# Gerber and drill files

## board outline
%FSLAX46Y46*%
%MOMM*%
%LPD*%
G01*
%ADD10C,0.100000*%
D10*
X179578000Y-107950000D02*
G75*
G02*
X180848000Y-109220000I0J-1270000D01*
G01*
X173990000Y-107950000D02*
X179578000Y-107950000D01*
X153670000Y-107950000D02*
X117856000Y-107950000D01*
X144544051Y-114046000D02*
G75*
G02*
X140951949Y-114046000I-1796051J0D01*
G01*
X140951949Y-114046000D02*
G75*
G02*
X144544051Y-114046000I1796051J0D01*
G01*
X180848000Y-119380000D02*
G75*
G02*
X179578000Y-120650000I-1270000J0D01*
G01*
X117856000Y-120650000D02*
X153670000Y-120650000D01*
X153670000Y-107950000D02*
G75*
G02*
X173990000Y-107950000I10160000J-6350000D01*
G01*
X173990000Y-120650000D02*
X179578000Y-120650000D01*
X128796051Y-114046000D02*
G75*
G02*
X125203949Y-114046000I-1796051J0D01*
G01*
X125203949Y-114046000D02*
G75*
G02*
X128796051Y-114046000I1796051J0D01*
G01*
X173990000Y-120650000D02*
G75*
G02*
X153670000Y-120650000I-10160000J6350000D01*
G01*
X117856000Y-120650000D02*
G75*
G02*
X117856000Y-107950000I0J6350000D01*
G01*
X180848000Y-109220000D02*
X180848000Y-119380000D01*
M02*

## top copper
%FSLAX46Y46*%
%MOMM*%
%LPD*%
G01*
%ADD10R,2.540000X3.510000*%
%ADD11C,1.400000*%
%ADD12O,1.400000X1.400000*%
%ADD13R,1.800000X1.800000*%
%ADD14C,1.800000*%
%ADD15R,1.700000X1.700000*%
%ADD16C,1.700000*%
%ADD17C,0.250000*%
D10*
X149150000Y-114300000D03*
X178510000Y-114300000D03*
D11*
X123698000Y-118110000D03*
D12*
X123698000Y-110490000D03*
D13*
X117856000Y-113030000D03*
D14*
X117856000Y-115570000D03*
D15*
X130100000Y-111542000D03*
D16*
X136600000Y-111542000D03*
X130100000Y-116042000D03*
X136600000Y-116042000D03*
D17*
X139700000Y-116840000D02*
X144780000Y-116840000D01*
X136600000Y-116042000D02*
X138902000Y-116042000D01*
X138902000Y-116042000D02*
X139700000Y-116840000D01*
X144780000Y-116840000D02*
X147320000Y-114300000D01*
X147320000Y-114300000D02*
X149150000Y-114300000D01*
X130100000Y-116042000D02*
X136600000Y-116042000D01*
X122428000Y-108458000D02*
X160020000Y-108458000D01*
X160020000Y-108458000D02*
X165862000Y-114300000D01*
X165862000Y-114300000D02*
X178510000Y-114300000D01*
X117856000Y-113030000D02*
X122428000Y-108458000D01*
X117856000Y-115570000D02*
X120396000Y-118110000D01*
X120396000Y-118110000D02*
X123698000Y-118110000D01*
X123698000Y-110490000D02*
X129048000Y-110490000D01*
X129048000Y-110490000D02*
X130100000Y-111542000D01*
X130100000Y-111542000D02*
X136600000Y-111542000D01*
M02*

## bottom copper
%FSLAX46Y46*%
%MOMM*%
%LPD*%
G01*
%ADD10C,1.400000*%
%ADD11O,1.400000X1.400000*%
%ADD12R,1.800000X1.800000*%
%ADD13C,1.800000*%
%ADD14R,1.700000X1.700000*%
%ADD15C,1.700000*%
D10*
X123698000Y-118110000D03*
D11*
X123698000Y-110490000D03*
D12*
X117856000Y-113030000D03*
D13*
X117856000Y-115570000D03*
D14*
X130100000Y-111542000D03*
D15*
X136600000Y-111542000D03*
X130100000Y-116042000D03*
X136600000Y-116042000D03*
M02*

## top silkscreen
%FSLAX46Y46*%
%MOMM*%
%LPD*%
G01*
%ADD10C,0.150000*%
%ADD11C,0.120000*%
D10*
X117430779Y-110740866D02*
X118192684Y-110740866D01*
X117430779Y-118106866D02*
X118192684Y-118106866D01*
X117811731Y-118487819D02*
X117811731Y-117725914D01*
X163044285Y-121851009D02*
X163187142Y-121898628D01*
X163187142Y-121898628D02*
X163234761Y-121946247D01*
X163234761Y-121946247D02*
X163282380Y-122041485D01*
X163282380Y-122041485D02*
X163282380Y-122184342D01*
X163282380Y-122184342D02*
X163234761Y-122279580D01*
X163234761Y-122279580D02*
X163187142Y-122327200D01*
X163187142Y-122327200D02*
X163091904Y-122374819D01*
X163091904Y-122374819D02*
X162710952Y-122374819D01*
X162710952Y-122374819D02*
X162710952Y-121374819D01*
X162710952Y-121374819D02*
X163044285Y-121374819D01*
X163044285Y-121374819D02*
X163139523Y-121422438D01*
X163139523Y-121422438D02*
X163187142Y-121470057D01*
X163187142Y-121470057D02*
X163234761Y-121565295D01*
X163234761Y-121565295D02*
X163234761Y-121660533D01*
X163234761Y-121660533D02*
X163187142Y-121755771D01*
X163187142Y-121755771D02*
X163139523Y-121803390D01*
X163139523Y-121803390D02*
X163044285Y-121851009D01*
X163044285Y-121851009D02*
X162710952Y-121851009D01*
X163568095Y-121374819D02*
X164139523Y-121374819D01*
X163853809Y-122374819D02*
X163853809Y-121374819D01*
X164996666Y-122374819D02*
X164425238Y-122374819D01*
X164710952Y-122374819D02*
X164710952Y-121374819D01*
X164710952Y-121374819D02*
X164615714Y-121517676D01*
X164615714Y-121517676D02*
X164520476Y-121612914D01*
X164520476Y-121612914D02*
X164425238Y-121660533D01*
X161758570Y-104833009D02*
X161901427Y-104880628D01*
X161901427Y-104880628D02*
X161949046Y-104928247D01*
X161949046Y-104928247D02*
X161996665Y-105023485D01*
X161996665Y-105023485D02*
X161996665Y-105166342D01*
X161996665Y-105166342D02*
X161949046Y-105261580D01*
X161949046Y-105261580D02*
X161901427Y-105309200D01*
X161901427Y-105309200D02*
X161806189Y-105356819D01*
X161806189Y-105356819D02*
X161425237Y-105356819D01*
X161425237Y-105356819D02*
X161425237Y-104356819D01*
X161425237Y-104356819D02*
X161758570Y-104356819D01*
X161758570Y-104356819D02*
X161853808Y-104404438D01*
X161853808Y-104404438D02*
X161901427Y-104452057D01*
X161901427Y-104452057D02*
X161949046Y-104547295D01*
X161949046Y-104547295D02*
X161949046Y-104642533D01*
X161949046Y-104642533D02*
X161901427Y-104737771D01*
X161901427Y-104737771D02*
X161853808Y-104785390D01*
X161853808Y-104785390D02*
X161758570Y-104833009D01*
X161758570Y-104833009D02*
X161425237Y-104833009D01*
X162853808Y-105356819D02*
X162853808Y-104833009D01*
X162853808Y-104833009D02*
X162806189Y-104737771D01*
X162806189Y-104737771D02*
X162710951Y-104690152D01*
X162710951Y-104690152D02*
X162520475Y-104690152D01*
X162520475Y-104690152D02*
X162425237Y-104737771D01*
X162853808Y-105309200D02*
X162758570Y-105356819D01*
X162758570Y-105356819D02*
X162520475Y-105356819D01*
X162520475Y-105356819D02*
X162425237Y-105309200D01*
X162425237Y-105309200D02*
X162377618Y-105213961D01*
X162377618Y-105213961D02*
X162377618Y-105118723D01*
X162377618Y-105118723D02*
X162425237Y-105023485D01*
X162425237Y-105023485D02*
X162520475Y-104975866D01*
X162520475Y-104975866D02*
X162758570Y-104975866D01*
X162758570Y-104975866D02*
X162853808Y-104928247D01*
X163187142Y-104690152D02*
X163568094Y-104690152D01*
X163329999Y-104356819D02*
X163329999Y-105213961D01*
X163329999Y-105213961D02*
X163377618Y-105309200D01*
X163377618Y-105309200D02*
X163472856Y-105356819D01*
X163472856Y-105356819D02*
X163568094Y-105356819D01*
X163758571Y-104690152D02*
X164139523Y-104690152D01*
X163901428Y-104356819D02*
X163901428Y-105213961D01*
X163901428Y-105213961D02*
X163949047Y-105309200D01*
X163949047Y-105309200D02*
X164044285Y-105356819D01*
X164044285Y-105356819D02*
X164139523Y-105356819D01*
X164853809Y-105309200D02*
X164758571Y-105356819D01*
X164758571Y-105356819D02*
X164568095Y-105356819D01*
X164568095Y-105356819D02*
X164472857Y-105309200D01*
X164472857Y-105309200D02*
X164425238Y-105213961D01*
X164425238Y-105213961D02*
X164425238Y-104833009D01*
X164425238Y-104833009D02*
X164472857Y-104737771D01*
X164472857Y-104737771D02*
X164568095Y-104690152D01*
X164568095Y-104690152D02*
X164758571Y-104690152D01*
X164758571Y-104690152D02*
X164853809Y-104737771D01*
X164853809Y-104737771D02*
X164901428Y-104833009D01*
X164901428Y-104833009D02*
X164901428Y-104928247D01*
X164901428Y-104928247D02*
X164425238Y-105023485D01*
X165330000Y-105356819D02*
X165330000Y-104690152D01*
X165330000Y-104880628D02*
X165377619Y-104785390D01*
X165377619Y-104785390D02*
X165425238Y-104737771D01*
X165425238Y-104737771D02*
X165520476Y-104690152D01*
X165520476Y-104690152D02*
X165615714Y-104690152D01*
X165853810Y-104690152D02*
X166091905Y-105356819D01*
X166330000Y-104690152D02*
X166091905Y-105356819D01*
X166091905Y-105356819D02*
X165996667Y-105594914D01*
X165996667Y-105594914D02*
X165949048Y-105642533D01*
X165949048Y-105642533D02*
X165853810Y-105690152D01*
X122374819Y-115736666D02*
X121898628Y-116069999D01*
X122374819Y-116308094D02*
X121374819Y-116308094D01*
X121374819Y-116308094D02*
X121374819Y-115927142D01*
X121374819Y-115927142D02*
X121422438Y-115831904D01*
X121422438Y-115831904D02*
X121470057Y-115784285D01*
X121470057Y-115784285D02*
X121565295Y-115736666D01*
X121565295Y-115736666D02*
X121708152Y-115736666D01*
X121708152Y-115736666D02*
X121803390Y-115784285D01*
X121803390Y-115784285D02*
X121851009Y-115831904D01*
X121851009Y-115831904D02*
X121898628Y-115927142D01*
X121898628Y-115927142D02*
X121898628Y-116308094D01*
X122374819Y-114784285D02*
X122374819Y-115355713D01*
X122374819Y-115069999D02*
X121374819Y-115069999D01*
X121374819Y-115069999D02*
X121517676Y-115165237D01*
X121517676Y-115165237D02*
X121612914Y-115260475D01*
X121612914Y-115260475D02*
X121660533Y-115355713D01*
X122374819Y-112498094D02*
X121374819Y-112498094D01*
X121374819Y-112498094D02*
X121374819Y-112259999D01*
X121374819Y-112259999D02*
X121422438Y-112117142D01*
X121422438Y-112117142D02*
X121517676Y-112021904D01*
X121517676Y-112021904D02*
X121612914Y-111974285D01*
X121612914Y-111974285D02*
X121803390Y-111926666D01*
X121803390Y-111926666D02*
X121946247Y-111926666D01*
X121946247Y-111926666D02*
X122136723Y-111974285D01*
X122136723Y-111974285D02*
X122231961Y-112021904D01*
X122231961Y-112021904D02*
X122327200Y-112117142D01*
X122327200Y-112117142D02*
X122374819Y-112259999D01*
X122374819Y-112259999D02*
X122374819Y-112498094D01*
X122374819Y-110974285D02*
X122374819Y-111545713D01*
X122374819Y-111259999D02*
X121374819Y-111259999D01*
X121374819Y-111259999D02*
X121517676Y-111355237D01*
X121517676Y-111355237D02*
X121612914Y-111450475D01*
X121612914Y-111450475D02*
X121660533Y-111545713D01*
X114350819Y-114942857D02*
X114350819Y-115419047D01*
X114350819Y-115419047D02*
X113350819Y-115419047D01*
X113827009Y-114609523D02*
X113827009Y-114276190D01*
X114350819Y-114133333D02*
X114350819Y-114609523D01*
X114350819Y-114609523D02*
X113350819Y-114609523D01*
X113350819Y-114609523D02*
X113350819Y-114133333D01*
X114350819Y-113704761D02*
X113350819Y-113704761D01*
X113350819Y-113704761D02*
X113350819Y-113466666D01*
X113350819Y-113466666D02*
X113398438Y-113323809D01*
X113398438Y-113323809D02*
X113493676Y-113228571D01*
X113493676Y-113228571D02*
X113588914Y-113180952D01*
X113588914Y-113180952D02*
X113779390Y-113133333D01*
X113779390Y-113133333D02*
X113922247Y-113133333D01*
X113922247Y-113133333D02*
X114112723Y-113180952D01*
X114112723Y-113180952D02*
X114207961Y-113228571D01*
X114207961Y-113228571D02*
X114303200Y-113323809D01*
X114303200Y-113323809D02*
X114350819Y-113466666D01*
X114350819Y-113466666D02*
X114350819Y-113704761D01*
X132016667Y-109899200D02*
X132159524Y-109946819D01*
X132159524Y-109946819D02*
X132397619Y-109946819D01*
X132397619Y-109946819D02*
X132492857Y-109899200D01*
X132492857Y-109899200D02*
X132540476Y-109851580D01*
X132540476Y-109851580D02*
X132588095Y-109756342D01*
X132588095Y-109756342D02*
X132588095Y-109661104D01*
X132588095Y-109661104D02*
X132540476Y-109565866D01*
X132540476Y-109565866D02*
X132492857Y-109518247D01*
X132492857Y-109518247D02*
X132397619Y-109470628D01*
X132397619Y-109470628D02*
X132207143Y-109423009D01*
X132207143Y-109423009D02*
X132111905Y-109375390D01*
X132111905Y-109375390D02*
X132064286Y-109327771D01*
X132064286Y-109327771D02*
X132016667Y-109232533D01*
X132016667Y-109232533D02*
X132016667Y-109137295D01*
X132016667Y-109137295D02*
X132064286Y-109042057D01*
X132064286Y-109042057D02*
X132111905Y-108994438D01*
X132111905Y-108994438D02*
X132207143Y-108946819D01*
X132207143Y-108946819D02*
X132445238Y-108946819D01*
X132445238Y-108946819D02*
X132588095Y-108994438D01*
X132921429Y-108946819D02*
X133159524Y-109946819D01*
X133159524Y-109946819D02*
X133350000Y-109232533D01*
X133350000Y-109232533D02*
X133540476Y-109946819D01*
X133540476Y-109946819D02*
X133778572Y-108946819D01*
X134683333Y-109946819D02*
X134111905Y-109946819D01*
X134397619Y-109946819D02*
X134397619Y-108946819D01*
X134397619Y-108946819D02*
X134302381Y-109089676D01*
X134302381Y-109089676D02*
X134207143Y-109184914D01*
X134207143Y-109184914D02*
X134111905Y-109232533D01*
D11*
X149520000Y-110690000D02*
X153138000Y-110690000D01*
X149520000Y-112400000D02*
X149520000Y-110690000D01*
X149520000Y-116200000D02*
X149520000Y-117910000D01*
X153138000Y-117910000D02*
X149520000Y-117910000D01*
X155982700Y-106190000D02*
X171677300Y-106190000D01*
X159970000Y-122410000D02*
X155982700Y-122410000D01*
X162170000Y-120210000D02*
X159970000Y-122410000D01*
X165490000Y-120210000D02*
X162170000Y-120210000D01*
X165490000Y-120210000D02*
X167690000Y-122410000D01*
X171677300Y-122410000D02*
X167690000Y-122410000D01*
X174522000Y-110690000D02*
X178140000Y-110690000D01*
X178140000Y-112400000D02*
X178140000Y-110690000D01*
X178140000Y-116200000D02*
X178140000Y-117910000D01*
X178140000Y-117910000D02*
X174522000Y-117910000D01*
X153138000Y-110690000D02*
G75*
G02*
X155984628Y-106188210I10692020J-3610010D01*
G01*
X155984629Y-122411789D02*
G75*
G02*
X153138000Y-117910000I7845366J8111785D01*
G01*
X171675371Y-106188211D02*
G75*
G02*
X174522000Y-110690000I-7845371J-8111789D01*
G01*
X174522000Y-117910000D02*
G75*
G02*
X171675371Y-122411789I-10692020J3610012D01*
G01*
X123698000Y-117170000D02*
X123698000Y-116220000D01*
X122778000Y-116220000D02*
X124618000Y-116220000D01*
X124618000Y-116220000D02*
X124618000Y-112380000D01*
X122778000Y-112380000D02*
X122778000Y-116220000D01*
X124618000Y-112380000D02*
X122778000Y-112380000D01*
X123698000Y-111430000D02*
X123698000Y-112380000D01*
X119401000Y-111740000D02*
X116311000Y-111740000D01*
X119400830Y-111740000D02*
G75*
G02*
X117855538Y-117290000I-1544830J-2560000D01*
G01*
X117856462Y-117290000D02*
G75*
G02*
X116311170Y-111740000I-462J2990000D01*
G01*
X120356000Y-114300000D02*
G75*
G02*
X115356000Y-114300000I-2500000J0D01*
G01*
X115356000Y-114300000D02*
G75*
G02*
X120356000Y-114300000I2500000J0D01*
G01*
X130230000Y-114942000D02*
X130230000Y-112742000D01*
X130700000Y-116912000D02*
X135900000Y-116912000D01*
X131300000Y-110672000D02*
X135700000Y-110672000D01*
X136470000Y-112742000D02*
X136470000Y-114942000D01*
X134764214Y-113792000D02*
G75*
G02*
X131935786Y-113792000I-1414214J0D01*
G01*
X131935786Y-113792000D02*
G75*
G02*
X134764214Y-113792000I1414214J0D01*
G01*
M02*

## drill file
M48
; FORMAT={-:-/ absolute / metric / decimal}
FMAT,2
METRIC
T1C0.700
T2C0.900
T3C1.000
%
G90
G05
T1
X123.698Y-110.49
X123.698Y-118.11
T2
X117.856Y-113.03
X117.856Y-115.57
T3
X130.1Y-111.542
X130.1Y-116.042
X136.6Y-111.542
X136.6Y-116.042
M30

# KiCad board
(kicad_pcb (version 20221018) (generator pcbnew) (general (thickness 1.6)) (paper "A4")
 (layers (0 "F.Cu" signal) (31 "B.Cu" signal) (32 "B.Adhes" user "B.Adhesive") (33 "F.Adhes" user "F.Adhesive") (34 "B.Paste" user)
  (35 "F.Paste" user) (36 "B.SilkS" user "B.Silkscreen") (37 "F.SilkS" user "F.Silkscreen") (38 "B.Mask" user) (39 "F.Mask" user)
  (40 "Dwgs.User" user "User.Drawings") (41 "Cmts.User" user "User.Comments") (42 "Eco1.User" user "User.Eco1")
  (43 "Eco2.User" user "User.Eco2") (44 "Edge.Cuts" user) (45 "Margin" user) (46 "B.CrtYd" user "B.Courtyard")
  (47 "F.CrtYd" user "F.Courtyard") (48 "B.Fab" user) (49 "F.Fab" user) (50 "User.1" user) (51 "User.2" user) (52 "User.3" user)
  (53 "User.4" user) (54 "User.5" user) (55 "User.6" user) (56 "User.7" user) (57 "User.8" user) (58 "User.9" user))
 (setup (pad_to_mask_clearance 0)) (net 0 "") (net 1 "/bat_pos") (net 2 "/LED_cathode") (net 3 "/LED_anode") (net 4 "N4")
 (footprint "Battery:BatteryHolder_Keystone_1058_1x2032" (layer "F.Cu") (at 163.83 114.3)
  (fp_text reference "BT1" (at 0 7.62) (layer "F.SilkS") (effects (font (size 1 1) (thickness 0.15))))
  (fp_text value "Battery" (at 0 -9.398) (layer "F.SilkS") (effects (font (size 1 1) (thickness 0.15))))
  (fp_line (start -14.31 -3.61) (end -10.692 -3.61) (stroke (width 0.12) (type solid)) (layer "F.SilkS"))
  (fp_line (start -14.31 -1.9) (end -14.31 -3.61) (stroke (width 0.12) (type solid)) (layer "F.SilkS"))
  (fp_line (start -14.31 1.9) (end -14.31 3.61) (stroke (width 0.12) (type solid)) (layer "F.SilkS"))
  (fp_line (start -10.692 3.61) (end -14.31 3.61) (stroke (width 0.12) (type solid)) (layer "F.SilkS"))
  (fp_line (start -7.8473 -8.11) (end 7.8473 -8.11) (stroke (width 0.12) (type solid)) (layer "F.SilkS"))
  (fp_line (start -3.86 8.11) (end -7.8473 8.11) (stroke (width 0.12) (type solid)) (layer "F.SilkS"))
  (fp_line (start -1.66 5.91) (end -3.86 8.11) (stroke (width 0.12) (type solid)) (layer "F.SilkS"))
  (fp_line (start 1.66 5.91) (end -1.66 5.91) (stroke (width 0.12) (type solid)) (layer "F.SilkS"))
  (fp_line (start 1.66 5.91) (end 3.86 8.11) (stroke (width 0.12) (type solid)) (layer "F.SilkS"))
  (fp_line (start 7.8473 8.11) (end 3.86 8.11) (stroke (width 0.12) (type solid)) (layer "F.SilkS"))
  (fp_line (start 10.692 -3.61) (end 14.31 -3.61) (stroke (width 0.12) (type solid)) (layer "F.SilkS"))
  (fp_line (start 14.31 -1.9) (end 14.31 -3.61) (stroke (width 0.12) (type solid)) (layer "F.SilkS"))
  (fp_line (start 14.31 1.9) (end 14.31 3.61) (stroke (width 0.12) (type solid)) (layer "F.SilkS"))
  (fp_line (start 14.31 3.61) (end 10.692 3.61) (stroke (width 0.12) (type solid)) (layer "F.SilkS"))
  (fp_arc (start -10.692 -3.61) (mid -9.538084 -6.031244) (end -7.845371 -8.111789) (stroke (width 0.12) (type solid)) (layer "F.SilkS"))
  (fp_arc (start -7.845371 8.111789) (mid -9.538085 6.031244) (end -10.692 3.61) (stroke (width 0.12) (type solid)) (layer "F.SilkS"))
  (fp_arc (start 7.845371 -8.111789) (mid 9.538085 -6.031244) (end 10.692 -3.61) (stroke (width 0.12) (type solid)) (layer "F.SilkS"))
  (fp_arc (start 10.692 3.61) (mid 9.538084 6.031244) (end 7.845371 8.111789) (stroke (width 0.12) (type solid)) (layer "F.SilkS"))
  (pad "1" smd rect (at -14.68 0) (size 2.54 3.51) (layers "F.Cu" "F.Paste" "F.Mask") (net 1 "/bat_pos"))
  (pad "2" smd rect (at 14.68 0) (size 2.54 3.51) (layers "F.Cu" "F.Paste" "F.Mask") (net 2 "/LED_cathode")))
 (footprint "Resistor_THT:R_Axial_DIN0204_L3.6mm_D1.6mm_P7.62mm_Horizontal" (layer "F.Cu") (at 123.698 118.11 90)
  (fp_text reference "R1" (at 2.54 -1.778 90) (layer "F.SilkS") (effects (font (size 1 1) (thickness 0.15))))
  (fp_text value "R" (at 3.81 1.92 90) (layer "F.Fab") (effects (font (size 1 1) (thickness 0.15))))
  (fp_line (start 0.94 0) (end 1.89 0) (stroke (width 0.12) (type solid)) (layer "F.SilkS"))
  (fp_line (start 1.89 -0.92) (end 1.89 0.92) (stroke (width 0.12) (type solid)) (layer "F.SilkS"))
  (fp_line (start 1.89 0.92) (end 5.73 0.92) (stroke (width 0.12) (type solid)) (layer "F.SilkS"))
  (fp_line (start 5.73 -0.92) (end 1.89 -0.92) (stroke (width 0.12) (type solid)) (layer "F.SilkS"))
  (fp_line (start 5.73 0.92) (end 5.73 -0.92) (stroke (width 0.12) (type solid)) (layer "F.SilkS"))
  (fp_line (start 6.68 0) (end 5.73 0) (stroke (width 0.12) (type solid)) (layer "F.SilkS"))
  (pad "1" thru_hole circle (at 0 0 90) (size 1.4 1.4) (drill 0.7) (layers "*.Cu" "*.Mask") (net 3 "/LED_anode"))
  (pad "2" thru_hole oval (at 7.62 0 90) (size 1.4 1.4) (drill 0.7) (layers "*.Cu" "*.Mask") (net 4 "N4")))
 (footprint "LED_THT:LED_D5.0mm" (layer "F.Cu") (at 117.856 113.03 -90)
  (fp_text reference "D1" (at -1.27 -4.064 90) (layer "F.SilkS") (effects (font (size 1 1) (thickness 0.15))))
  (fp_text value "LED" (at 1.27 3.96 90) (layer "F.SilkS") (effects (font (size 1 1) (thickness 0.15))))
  (fp_line (start -1.29 -1.545) (end -1.29 1.545) (stroke (width 0.12) (type solid)) (layer "F.SilkS"))
  (fp_arc (start -1.29 -1.54483) (mid 2.072002 -2.880433) (end 4.26 0.000462) (stroke (width 0.12) (type solid)) (layer "F.SilkS"))
  (fp_arc (start 4.26 -0.000462) (mid 2.072002 2.880433) (end -1.29 1.54483) (stroke (width 0.12) (type solid)) (layer "F.SilkS"))
  (fp_circle (center 1.27 0) (end 3.77 0) (stroke (width 0.12) (type solid)) (fill none) (layer "F.SilkS"))
  (pad "1" thru_hole rect (at 0 0 270) (size 1.8 1.8) (drill 0.9) (layers "*.Cu" "*.Mask") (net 2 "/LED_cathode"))
  (pad "2" thru_hole circle (at 2.54 0 270) (size 1.8 1.8) (drill 0.9) (layers "*.Cu" "*.Mask") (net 3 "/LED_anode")))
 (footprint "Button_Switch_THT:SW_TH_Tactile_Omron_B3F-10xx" (layer "F.Cu") (at 130.1 111.542)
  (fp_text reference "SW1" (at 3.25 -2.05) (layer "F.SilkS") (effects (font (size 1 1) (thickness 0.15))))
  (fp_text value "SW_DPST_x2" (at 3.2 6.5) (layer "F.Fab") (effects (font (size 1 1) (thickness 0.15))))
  (fp_line (start 0.13 3.4) (end 0.13 1.2) (stroke (width 0.12) (type solid)) (layer "F.SilkS"))
  (fp_line (start 0.6 5.37) (end 5.8 5.37) (stroke (width 0.12) (type solid)) (layer "F.SilkS"))
  (fp_line (start 1.2 -0.87) (end 5.6 -0.87) (stroke (width 0.12) (type solid)) (layer "F.SilkS"))
  (fp_line (start 6.37 1.2) (end 6.37 3.4) (stroke (width 0.12) (type solid)) (layer "F.SilkS"))
  (fp_circle (center 3.25 2.25) (end 4.25 3.25) (stroke (width 0.12) (type solid)) (fill none) (layer "F.SilkS"))
  (pad "1" thru_hole rect (at 0 0) (size 1.7 1.7) (drill 1) (layers "*.Cu" "*.Mask") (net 4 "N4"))
  (pad "1" thru_hole circle (at 6.5 0) (size 1.7 1.7) (drill 1) (layers "*.Cu" "*.Mask") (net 4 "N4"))
  (pad "2" thru_hole circle (at 0 4.5) (size 1.7 1.7) (drill 1) (layers "*.Cu" "*.Mask") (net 1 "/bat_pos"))
  (pad "2" thru_hole circle (at 6.5 4.5) (size 1.7 1.7) (drill 1) (layers "*.Cu" "*.Mask") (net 1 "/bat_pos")))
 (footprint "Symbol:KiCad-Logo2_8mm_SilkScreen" (layer "B.Cu") (at 163.83 114.3 180)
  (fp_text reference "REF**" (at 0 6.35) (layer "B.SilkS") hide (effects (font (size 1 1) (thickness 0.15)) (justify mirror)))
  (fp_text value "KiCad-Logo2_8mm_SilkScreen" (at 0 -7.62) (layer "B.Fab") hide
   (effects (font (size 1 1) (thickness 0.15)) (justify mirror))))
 (gr_arc (start 179.578 107.95) (mid 180.476026 108.321974) (end 180.848 109.22) (stroke (width 0.1) (type default)) (layer "Edge.Cuts"))
 (gr_line (start 173.99 107.95) (end 179.578 107.95) (stroke (width 0.1) (type default)) (layer "Edge.Cuts"))
 (gr_line (start 153.67 107.95) (end 117.856 107.95) (stroke (width 0.1) (type default)) (layer "Edge.Cuts"))
 (gr_circle (center 142.748 114.046) (end 141.478 112.776) (stroke (width 0.1) (type default)) (fill none) (layer "Edge.Cuts"))
 (gr_arc (start 180.848 119.38) (mid 180.476026 120.278026) (end 179.578 120.65) (stroke (width 0.1) (type default)) (layer "Edge.Cuts"))
 (gr_line (start 117.856 120.65) (end 153.67 120.65) (stroke (width 0.1) (type default)) (layer "Edge.Cuts"))
 (gr_arc (start 153.67 107.95) (mid 163.83 102.318844) (end 173.99 107.95) (stroke (width 0.1) (type default)) (layer "Edge.Cuts"))
 (gr_line (start 173.99 120.65) (end 179.578 120.65) (stroke (width 0.1) (type default)) (layer "Edge.Cuts"))
 (gr_circle (center 127 114.046) (end 125.73 112.776) (stroke (width 0.1) (type default)) (fill none) (layer "Edge.Cuts"))
 (gr_arc (start 173.99 120.65) (mid 163.83 126.281156) (end 153.67 120.65) (stroke (width 0.1) (type default)) (layer "Edge.Cuts"))
 (gr_arc (start 117.856 120.65) (mid 111.506 114.3) (end 117.856 107.95) (stroke (width 0.1) (type default)) (layer "Edge.Cuts"))
 (gr_line (start 180.848 109.22) (end 180.848 119.38) (stroke (width 0.1) (type default)) (layer "Edge.Cuts"))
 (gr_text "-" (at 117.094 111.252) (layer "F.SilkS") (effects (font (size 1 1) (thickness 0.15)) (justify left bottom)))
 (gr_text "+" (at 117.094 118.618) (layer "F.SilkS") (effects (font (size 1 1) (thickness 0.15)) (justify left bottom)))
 (segment (start 139.7 116.84) (end 144.78 116.84) (width 0.25) (layer "F.Cu") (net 1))
 (segment (start 136.6 116.042) (end 138.902 116.042) (width 0.25) (layer "F.Cu") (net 1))
 (segment (start 138.902 116.042) (end 139.7 116.84) (width 0.25) (layer "F.Cu") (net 1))
 (segment (start 144.78 116.84) (end 147.32 114.3) (width 0.25) (layer "F.Cu") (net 1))
 (segment (start 147.32 114.3) (end 149.15 114.3) (width 0.25) (layer "F.Cu") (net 1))
 (segment (start 130.1 116.042) (end 136.6 116.042) (width 0.25) (layer "F.Cu") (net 1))
 (segment (start 122.428 108.458) (end 160.02 108.458) (width 0.25) (layer "F.Cu") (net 2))
 (segment (start 160.02 108.458) (end 165.862 114.3) (width 0.25) (layer "F.Cu") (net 2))
 (segment (start 165.862 114.3) (end 178.51 114.3) (width 0.25) (layer "F.Cu") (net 2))
 (segment (start 117.856 113.03) (end 122.428 108.458) (width 0.25) (layer "F.Cu") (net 2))
 (segment (start 117.856 115.57) (end 120.396 118.11) (width 0.25) (layer "F.Cu") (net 3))
 (segment (start 120.396 118.11) (end 123.698 118.11) (width 0.25) (layer "F.Cu") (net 3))
 (segment (start 123.698 110.49) (end 129.048 110.49) (width 0.25) (layer "F.Cu") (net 4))
 (segment (start 129.048 110.49) (end 130.1 111.542) (width 0.25) (layer "F.Cu") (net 4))
 (segment (start 130.1 111.542) (end 136.6 111.542) (width 0.25) (layer "F.Cu") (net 4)))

